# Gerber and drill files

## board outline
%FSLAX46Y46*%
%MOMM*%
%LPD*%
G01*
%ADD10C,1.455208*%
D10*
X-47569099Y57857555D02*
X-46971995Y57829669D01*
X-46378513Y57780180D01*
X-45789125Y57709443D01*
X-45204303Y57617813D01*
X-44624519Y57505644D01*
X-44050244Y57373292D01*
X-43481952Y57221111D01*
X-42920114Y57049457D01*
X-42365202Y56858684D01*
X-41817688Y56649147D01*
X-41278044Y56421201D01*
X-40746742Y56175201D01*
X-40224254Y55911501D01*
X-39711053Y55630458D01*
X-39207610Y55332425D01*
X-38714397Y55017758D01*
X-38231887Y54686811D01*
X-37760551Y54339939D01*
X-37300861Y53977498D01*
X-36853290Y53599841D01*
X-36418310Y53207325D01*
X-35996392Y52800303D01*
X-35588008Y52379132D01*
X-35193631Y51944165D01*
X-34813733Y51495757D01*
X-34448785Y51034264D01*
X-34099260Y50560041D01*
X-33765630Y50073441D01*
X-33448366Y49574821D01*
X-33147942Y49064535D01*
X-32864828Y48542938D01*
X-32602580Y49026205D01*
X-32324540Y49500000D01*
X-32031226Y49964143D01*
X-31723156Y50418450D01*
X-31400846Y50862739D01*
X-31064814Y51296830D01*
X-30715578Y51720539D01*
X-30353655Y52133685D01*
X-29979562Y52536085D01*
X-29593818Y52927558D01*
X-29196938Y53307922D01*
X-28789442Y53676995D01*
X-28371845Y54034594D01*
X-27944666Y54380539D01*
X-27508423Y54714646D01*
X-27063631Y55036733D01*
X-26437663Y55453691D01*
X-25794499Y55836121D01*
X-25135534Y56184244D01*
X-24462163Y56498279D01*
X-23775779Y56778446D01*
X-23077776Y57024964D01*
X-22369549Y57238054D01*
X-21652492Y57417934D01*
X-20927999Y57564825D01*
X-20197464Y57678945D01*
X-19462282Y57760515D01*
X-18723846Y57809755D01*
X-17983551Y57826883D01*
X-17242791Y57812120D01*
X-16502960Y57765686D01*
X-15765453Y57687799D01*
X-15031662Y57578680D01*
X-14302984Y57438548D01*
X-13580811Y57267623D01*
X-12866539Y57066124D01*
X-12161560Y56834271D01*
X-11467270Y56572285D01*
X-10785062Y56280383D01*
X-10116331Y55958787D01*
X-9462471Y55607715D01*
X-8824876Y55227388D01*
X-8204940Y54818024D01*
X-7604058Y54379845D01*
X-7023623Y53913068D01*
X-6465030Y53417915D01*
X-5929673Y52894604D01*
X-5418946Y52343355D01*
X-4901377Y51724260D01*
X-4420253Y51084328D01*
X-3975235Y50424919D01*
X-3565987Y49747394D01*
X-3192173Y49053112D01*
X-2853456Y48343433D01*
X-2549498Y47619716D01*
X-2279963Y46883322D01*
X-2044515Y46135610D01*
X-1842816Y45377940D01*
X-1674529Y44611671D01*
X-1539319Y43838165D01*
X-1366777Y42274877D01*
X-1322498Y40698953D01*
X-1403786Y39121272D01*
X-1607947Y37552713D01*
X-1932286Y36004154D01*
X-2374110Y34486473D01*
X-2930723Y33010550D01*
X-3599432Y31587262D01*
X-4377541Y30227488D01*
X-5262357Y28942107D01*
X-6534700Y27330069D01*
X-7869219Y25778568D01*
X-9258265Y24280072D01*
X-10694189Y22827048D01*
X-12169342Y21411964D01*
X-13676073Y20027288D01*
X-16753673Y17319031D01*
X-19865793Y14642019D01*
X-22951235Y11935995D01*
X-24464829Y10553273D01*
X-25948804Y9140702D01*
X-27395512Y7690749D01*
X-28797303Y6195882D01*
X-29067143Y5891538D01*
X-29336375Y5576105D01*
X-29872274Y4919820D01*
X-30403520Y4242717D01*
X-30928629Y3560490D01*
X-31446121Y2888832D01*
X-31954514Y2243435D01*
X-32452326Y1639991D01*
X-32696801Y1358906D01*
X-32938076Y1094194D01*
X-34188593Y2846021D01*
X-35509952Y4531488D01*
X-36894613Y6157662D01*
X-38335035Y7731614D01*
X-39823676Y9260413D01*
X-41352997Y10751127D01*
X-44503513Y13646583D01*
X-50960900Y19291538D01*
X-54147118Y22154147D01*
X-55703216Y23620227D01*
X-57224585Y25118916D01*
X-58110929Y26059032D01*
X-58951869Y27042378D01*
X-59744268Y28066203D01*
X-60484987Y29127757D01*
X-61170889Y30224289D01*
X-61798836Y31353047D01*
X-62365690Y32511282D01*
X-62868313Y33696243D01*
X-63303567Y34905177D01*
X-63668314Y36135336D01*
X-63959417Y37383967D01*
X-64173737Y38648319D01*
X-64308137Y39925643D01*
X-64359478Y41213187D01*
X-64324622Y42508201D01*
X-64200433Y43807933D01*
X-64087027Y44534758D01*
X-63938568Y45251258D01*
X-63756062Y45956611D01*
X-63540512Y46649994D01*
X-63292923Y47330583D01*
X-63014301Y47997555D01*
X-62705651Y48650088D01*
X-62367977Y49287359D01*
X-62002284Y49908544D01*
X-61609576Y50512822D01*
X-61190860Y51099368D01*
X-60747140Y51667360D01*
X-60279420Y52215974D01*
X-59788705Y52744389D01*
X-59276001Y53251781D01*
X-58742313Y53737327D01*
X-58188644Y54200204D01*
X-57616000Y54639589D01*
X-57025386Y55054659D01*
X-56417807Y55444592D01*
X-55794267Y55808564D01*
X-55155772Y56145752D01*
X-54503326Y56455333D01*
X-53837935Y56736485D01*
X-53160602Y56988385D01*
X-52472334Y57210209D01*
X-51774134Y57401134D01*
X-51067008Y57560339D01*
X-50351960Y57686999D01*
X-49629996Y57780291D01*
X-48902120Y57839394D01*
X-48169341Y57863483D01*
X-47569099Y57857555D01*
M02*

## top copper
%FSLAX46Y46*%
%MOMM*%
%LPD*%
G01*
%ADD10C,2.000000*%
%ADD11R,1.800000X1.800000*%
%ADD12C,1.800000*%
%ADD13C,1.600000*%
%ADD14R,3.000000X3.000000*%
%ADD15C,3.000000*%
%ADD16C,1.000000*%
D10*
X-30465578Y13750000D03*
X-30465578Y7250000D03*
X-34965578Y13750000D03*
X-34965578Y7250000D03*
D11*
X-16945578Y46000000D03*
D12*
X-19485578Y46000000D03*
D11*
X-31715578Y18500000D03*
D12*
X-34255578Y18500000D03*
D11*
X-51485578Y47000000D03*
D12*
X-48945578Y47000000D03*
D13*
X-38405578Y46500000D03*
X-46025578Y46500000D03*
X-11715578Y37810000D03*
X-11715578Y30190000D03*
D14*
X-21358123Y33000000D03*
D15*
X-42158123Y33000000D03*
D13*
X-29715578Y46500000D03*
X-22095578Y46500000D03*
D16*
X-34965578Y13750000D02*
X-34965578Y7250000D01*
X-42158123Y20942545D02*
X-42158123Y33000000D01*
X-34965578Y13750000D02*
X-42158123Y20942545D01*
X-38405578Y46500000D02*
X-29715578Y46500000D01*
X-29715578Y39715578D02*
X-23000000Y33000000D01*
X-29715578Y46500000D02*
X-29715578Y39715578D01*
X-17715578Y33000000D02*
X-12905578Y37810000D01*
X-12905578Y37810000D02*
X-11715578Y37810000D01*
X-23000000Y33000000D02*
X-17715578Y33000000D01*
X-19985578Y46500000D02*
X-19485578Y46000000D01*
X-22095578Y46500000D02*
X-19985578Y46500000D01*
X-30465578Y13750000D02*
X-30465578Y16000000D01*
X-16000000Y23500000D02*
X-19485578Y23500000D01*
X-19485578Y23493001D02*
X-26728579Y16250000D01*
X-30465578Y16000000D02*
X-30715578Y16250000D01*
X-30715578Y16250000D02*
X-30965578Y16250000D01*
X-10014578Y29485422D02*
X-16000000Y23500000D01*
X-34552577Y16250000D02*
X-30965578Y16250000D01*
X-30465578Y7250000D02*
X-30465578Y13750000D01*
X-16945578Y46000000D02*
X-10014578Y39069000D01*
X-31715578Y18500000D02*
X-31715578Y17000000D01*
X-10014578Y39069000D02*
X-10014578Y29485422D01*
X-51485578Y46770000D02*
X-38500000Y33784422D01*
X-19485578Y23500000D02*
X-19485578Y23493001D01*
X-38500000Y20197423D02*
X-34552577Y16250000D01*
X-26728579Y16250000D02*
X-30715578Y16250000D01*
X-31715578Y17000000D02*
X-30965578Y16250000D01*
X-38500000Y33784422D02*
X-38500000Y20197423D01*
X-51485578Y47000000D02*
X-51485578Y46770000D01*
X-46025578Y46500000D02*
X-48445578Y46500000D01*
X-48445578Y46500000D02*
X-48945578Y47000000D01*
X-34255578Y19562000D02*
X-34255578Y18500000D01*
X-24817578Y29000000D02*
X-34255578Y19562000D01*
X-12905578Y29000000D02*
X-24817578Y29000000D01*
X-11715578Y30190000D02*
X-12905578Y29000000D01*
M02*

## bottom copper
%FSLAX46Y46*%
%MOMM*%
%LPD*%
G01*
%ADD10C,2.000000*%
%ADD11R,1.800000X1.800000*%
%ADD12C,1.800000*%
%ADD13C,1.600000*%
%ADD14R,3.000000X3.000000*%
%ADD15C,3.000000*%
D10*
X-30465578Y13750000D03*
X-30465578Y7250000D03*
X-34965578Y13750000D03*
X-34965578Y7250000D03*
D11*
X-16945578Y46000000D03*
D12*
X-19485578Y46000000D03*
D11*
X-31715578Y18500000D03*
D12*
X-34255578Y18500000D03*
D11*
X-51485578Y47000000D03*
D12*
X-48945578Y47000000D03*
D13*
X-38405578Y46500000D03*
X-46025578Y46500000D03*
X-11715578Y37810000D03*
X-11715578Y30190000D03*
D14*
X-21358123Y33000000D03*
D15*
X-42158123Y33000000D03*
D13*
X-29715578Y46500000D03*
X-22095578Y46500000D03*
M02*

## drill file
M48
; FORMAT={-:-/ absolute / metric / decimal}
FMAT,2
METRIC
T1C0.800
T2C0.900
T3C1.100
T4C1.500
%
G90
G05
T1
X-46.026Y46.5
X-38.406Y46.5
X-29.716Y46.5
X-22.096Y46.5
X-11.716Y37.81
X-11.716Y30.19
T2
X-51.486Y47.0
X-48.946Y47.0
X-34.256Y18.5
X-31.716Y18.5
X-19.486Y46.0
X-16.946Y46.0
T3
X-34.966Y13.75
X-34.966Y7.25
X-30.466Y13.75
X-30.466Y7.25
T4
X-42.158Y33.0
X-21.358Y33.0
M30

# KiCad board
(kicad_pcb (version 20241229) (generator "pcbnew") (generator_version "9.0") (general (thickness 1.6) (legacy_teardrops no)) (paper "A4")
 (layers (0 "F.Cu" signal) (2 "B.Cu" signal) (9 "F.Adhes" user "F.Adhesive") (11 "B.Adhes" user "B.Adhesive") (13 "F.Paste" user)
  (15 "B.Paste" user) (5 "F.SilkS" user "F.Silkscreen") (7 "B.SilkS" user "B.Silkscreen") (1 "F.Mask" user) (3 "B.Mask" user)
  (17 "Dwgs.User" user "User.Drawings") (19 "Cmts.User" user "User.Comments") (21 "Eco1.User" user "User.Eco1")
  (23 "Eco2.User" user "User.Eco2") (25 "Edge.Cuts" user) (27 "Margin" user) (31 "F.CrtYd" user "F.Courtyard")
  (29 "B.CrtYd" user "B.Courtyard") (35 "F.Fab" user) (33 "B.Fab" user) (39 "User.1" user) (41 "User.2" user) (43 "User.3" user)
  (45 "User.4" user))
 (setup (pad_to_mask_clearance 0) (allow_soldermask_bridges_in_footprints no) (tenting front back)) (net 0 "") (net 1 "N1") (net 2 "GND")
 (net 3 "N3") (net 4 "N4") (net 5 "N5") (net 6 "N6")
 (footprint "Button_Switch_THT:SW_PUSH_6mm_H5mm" (layer "F.Cu") (at -30.465578 -13.75 -90)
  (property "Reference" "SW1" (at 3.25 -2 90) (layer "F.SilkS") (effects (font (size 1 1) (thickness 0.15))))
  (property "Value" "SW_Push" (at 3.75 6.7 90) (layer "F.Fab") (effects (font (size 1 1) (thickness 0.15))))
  (pad "1" thru_hole circle (at 0 0) (size 2 2) (drill 1.1) (layers "*.Cu" "*.Mask") (remove_unused_layers no) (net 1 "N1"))
  (pad "1" thru_hole circle (at 6.5 0) (size 2 2) (drill 1.1) (layers "*.Cu" "*.Mask") (remove_unused_layers no) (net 1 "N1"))
  (pad "2" thru_hole circle (at 0 4.5) (size 2 2) (drill 1.1) (layers "*.Cu" "*.Mask") (remove_unused_layers no) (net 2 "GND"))
  (pad "2" thru_hole circle (at 6.5 4.5) (size 2 2) (drill 1.1) (layers "*.Cu" "*.Mask") (remove_unused_layers no) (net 2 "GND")))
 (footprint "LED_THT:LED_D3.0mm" (layer "F.Cu") (at -16.945578 -46 180)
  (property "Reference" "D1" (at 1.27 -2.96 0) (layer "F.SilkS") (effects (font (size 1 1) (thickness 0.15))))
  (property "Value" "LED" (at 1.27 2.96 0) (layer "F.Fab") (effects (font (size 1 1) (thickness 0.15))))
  (pad "1" thru_hole rect (at 0 0 180) (size 1.8 1.8) (drill 0.9) (layers "*.Cu" "*.Mask") (remove_unused_layers no) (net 1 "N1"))
  (pad "2" thru_hole circle (at 2.54 0 180) (size 1.8 1.8) (drill 0.9) (layers "*.Cu" "*.Mask") (remove_unused_layers no) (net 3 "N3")))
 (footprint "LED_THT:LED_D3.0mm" (layer "F.Cu") (at -31.715578 -18.5 180)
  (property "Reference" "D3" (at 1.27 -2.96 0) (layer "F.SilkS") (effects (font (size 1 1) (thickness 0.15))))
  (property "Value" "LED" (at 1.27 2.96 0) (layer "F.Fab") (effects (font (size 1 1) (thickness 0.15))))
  (pad "1" thru_hole rect (at 0 0 180) (size 1.8 1.8) (drill 0.9) (layers "*.Cu" "*.Mask") (remove_unused_layers no) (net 1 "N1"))
  (pad "2" thru_hole circle (at 2.54 0 180) (size 1.8 1.8) (drill 0.9) (layers "*.Cu" "*.Mask") (remove_unused_layers no) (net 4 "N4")))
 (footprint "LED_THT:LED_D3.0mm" (layer "F.Cu") (at -51.485578 -47)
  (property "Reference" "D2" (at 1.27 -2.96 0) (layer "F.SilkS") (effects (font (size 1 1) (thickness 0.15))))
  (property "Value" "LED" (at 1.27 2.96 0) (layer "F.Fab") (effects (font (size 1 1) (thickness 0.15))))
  (pad "1" thru_hole rect (at 0 0) (size 1.8 1.8) (drill 0.9) (layers "*.Cu" "*.Mask") (remove_unused_layers no) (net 1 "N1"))
  (pad "2" thru_hole circle (at 2.54 0) (size 1.8 1.8) (drill 0.9) (layers "*.Cu" "*.Mask") (remove_unused_layers no) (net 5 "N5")))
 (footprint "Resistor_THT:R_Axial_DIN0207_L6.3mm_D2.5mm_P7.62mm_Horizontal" (layer "B.Cu") (at -38.405578 -46.5 180)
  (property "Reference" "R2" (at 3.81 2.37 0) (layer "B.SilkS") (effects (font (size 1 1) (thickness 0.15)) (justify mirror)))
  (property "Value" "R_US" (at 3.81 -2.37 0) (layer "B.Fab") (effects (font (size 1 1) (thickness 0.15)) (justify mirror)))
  (pad "1" thru_hole circle (at 0 0 180) (size 1.6 1.6) (drill 0.8) (layers "*.Cu" "*.Mask") (remove_unused_layers no) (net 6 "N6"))
  (pad "2" thru_hole circle (at 7.62 0 180) (size 1.6 1.6) (drill 0.8) (layers "*.Cu" "*.Mask") (remove_unused_layers no) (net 5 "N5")))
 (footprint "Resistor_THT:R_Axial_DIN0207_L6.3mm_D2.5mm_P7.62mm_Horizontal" (layer "B.Cu") (at -11.715578 -37.81 -90)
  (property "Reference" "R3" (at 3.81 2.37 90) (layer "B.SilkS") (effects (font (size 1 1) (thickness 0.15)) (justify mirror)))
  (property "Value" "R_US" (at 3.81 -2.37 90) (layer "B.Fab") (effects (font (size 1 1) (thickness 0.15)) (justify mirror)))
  (pad "1" thru_hole circle (at 0 0 270) (size 1.6 1.6) (drill 0.8) (layers "*.Cu" "*.Mask") (remove_unused_layers no) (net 6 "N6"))
  (pad "2" thru_hole circle (at 7.62 0 270) (size 1.6 1.6) (drill 0.8) (layers "*.Cu" "*.Mask") (remove_unused_layers no) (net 4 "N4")))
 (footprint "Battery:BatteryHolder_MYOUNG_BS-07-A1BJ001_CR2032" (layer "B.Cu") (at -21.358123 -33 180)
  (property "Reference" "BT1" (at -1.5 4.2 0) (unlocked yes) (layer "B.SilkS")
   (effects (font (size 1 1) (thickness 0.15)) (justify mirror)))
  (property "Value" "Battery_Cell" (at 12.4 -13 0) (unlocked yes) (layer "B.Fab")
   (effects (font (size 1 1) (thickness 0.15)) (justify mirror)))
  (pad "1" thru_hole rect (at 0 0) (size 3 3) (drill 1.5) (layers "*.Cu" "*.Mask") (remove_unused_layers no) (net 6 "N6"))
  (pad "2" thru_hole circle (at 20.8 0) (size 3 3) (drill 1.5) (layers "*.Cu" "*.Mask") (remove_unused_layers no) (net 2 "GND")))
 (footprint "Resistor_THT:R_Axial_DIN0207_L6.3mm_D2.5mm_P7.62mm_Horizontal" (layer "B.Cu") (at -29.715578 -46.5)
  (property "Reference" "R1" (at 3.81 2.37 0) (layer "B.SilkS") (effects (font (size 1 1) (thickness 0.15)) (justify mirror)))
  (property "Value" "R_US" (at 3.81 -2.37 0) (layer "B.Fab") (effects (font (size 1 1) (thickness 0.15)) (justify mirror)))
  (pad "1" thru_hole circle (at 0 0) (size 1.6 1.6) (drill 0.8) (layers "*.Cu" "*.Mask") (remove_unused_layers no) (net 6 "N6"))
  (pad "2" thru_hole circle (at 7.62 0) (size 1.6 1.6) (drill 0.8) (layers "*.Cu" "*.Mask") (remove_unused_layers no) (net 3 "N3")))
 (gr_poly
  (pts (xy -47.569099 -57.857555) (xy -46.971995 -57.829669) (xy -46.378513 -57.78018) (xy -45.789125 -57.709443) (xy -45.204303 -57.617813)
   (xy -44.624519 -57.505644) (xy -44.050244 -57.373292) (xy -43.481952 -57.221111) (xy -42.920114 -57.049457) (xy -42.365202 -56.858684)
   (xy -41.817688 -56.649147) (xy -41.278044 -56.421201) (xy -40.746742 -56.175201) (xy -40.224254 -55.911501) (xy -39.711053 -55.630458)
   (xy -39.20761 -55.332425) (xy -38.714397 -55.017758) (xy -38.231887 -54.686811) (xy -37.760551 -54.339939) (xy -37.300861 -53.977498)
   (xy -36.85329 -53.599841) (xy -36.41831 -53.207325) (xy -35.996392 -52.800303) (xy -35.588008 -52.379132) (xy -35.193631 -51.944165)
   (xy -34.813733 -51.495757) (xy -34.448785 -51.034264) (xy -34.09926 -50.560041) (xy -33.76563 -50.073441) (xy -33.448366 -49.574821)
   (xy -33.147942 -49.064535) (xy -32.864828 -48.542938) (xy -32.60258 -49.026205) (xy -32.32454 -49.5) (xy -32.031226 -49.964143)
   (xy -31.723156 -50.41845) (xy -31.400846 -50.862739) (xy -31.064814 -51.29683) (xy -30.715578 -51.720539) (xy -30.353655 -52.133685)
   (xy -29.979562 -52.536085) (xy -29.593818 -52.927558) (xy -29.196938 -53.307922) (xy -28.789442 -53.676995) (xy -28.371845 -54.034594)
   (xy -27.944666 -54.380539) (xy -27.508423 -54.714646) (xy -27.063631 -55.036733) (xy -26.437663 -55.453691) (xy -25.794499 -55.836121)
   (xy -25.135534 -56.184244) (xy -24.462163 -56.498279) (xy -23.775779 -56.778446) (xy -23.077776 -57.024964) (xy -22.369549 -57.238054)
   (xy -21.652492 -57.417934) (xy -20.927999 -57.564825) (xy -20.197464 -57.678945) (xy -19.462282 -57.760515) (xy -18.723846 -57.809755)
   (xy -17.983551 -57.826883) (xy -17.242791 -57.81212) (xy -16.50296 -57.765686) (xy -15.765453 -57.687799) (xy -15.031662 -57.57868)
   (xy -14.302984 -57.438548) (xy -13.580811 -57.267623) (xy -12.866539 -57.066124) (xy -12.16156 -56.834271) (xy -11.46727 -56.572285)
   (xy -10.785062 -56.280383) (xy -10.116331 -55.958787) (xy -9.462471 -55.607715) (xy -8.824876 -55.227388) (xy -8.20494 -54.818024)
   (xy -7.604058 -54.379845) (xy -7.023623 -53.913068) (xy -6.46503 -53.417915) (xy -5.929673 -52.894604) (xy -5.418946 -52.343355)
   (xy -4.901377 -51.72426) (xy -4.420253 -51.084328) (xy -3.975235 -50.424919) (xy -3.565987 -49.747394) (xy -3.192173 -49.053112)
   (xy -2.853456 -48.343433) (xy -2.549498 -47.619716) (xy -2.279963 -46.883322) (xy -2.044515 -46.13561) (xy -1.842816 -45.37794)
   (xy -1.674529 -44.611671) (xy -1.539319 -43.838165) (xy -1.366777 -42.274877) (xy -1.322498 -40.698953) (xy -1.403786 -39.121272)
   (xy -1.607947 -37.552713) (xy -1.932286 -36.004154) (xy -2.37411 -34.486473) (xy -2.930723 -33.01055) (xy -3.599432 -31.587262)
   (xy -4.377541 -30.227488) (xy -5.262357 -28.942107) (xy -6.5347 -27.330069) (xy -7.869219 -25.778568) (xy -9.258265 -24.280072)
   (xy -10.694189 -22.827048) (xy -12.169342 -21.411964) (xy -13.676073 -20.027288) (xy -16.753673 -17.319031) (xy -19.865793 -14.642019)
   (xy -22.951235 -11.935995) (xy -24.464829 -10.553273) (xy -25.948804 -9.140702) (xy -27.395512 -7.690749) (xy -28.797303 -6.195882)
   (xy -29.067143 -5.891538) (xy -29.336375 -5.576105) (xy -29.872274 -4.91982) (xy -30.40352 -4.242717) (xy -30.928629 -3.56049)
   (xy -31.446121 -2.888832) (xy -31.954514 -2.243435) (xy -32.452326 -1.639991) (xy -32.696801 -1.358906) (xy -32.938076 -1.094194)
   (xy -34.188593 -2.846021) (xy -35.509952 -4.531488) (xy -36.894613 -6.157662) (xy -38.335035 -7.731614) (xy -39.823676 -9.260413)
   (xy -41.352997 -10.751127) (xy -44.503513 -13.646583) (xy -50.9609 -19.291538) (xy -54.147118 -22.154147) (xy -55.703216 -23.620227)
   (xy -57.224585 -25.118916) (xy -58.110929 -26.059032) (xy -58.951869 -27.042378) (xy -59.744268 -28.066203) (xy -60.484987 -29.127757)
   (xy -61.170889 -30.224289) (xy -61.798836 -31.353047) (xy -62.36569 -32.511282) (xy -62.868313 -33.696243) (xy -63.303567 -34.905177)
   (xy -63.668314 -36.135336) (xy -63.959417 -37.383967) (xy -64.173737 -38.648319) (xy -64.308137 -39.925643) (xy -64.359478 -41.213187)
   (xy -64.324622 -42.508201) (xy -64.200433 -43.807933) (xy -64.087027 -44.534758) (xy -63.938568 -45.251258) (xy -63.756062 -45.956611)
   (xy -63.540512 -46.649994) (xy -63.292923 -47.330583) (xy -63.014301 -47.997555) (xy -62.705651 -48.650088) (xy -62.367977 -49.287359)
   (xy -62.002284 -49.908544) (xy -61.609576 -50.512822) (xy -61.19086 -51.099368) (xy -60.74714 -51.66736) (xy -60.27942 -52.215974)
   (xy -59.788705 -52.744389) (xy -59.276001 -53.251781) (xy -58.742313 -53.737327) (xy -58.188644 -54.200204) (xy -57.616 -54.639589)
   (xy -57.025386 -55.054659) (xy -56.417807 -55.444592) (xy -55.794267 -55.808564) (xy -55.155772 -56.145752) (xy -54.503326 -56.455333)
   (xy -53.837935 -56.736485) (xy -53.160602 -56.988385) (xy -52.472334 -57.210209) (xy -51.774134 -57.401134) (xy -51.067008 -57.560339)
   (xy -50.35196 -57.686999) (xy -49.629996 -57.780291) (xy -48.90212 -57.839394) (xy -48.169341 -57.863483))
  (stroke (width 1.455208) (type solid)) (fill no) (layer "Edge.Cuts"))
 (segment (start -34.965578 -13.75) (end -34.965578 -7.25) (width 1) (layer "F.Cu") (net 2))
 (segment (start -42.158123 -20.942545) (end -42.158123 -33) (width 1) (layer "F.Cu") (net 2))
 (segment (start -34.965578 -13.75) (end -42.158123 -20.942545) (width 1) (layer "F.Cu") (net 2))
 (segment (start -38.405578 -46.5) (end -29.715578 -46.5) (width 1) (layer "F.Cu") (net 6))
 (segment (start -29.715578 -39.715578) (end -23 -33) (width 1) (layer "F.Cu") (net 6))
 (segment (start -29.715578 -46.5) (end -29.715578 -39.715578) (width 1) (layer "F.Cu") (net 6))
 (segment (start -17.715578 -33) (end -12.905578 -37.81) (width 1) (layer "F.Cu") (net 6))
 (segment (start -12.905578 -37.81) (end -11.715578 -37.81) (width 1) (layer "F.Cu") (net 6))
 (segment (start -23 -33) (end -17.715578 -33) (width 1) (layer "F.Cu") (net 6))
 (segment (start -19.985578 -46.5) (end -19.485578 -46) (width 1) (layer "F.Cu") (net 3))
 (segment (start -22.095578 -46.5) (end -19.985578 -46.5) (width 1) (layer "F.Cu") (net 3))
 (segment (start -30.465578 -13.75) (end -30.465578 -16) (width 1) (layer "F.Cu") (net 1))
 (segment (start -16 -23.5) (end -19.485578 -23.5) (width 1) (layer "F.Cu") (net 1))
 (segment (start -19.485578 -23.493001) (end -26.728579 -16.25) (width 1) (layer "F.Cu") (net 1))
 (segment (start -30.465578 -16) (end -30.715578 -16.25) (width 1) (layer "F.Cu") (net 1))
 (segment (start -30.715578 -16.25) (end -30.965578 -16.25) (width 1) (layer "F.Cu") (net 1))
 (segment (start -10.014578 -29.485422) (end -16 -23.5) (width 1) (layer "F.Cu") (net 1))
 (segment (start -34.552577 -16.25) (end -30.965578 -16.25) (width 1) (layer "F.Cu") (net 1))
 (segment (start -30.465578 -7.25) (end -30.465578 -13.75) (width 1) (layer "F.Cu") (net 1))
 (segment (start -16.945578 -46) (end -10.014578 -39.069) (width 1) (layer "F.Cu") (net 1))
 (segment (start -31.715578 -18.5) (end -31.715578 -17) (width 1) (layer "F.Cu") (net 1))
 (segment (start -10.014578 -39.069) (end -10.014578 -29.485422) (width 1) (layer "F.Cu") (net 1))
 (segment (start -51.485578 -46.77) (end -38.5 -33.784422) (width 1) (layer "F.Cu") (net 1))
 (segment (start -19.485578 -23.5) (end -19.485578 -23.493001) (width 1) (layer "F.Cu") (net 1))
 (segment (start -38.5 -20.197423) (end -34.552577 -16.25) (width 1) (layer "F.Cu") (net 1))
 (segment (start -26.728579 -16.25) (end -30.715578 -16.25) (width 1) (layer "F.Cu") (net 1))
 (segment (start -31.715578 -17) (end -30.965578 -16.25) (width 1) (layer "F.Cu") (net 1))
 (segment (start -38.5 -33.784422) (end -38.5 -20.197423) (width 1) (layer "F.Cu") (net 1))
 (segment (start -51.485578 -47) (end -51.485578 -46.77) (width 1) (layer "F.Cu") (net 1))
 (segment (start -46.025578 -46.5) (end -48.445578 -46.5) (width 1) (layer "F.Cu") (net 5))
 (segment (start -48.445578 -46.5) (end -48.945578 -47) (width 1) (layer "F.Cu") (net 5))
 (segment (start -34.255578 -19.562) (end -34.255578 -18.5) (width 1) (layer "F.Cu") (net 4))
 (segment (start -24.817578 -29) (end -34.255578 -19.562) (width 1) (layer "F.Cu") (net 4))
 (segment (start -12.905578 -29) (end -24.817578 -29) (width 1) (layer "F.Cu") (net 4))
 (segment (start -11.715578 -30.19) (end -12.905578 -29) (width 1) (layer "F.Cu") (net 4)))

